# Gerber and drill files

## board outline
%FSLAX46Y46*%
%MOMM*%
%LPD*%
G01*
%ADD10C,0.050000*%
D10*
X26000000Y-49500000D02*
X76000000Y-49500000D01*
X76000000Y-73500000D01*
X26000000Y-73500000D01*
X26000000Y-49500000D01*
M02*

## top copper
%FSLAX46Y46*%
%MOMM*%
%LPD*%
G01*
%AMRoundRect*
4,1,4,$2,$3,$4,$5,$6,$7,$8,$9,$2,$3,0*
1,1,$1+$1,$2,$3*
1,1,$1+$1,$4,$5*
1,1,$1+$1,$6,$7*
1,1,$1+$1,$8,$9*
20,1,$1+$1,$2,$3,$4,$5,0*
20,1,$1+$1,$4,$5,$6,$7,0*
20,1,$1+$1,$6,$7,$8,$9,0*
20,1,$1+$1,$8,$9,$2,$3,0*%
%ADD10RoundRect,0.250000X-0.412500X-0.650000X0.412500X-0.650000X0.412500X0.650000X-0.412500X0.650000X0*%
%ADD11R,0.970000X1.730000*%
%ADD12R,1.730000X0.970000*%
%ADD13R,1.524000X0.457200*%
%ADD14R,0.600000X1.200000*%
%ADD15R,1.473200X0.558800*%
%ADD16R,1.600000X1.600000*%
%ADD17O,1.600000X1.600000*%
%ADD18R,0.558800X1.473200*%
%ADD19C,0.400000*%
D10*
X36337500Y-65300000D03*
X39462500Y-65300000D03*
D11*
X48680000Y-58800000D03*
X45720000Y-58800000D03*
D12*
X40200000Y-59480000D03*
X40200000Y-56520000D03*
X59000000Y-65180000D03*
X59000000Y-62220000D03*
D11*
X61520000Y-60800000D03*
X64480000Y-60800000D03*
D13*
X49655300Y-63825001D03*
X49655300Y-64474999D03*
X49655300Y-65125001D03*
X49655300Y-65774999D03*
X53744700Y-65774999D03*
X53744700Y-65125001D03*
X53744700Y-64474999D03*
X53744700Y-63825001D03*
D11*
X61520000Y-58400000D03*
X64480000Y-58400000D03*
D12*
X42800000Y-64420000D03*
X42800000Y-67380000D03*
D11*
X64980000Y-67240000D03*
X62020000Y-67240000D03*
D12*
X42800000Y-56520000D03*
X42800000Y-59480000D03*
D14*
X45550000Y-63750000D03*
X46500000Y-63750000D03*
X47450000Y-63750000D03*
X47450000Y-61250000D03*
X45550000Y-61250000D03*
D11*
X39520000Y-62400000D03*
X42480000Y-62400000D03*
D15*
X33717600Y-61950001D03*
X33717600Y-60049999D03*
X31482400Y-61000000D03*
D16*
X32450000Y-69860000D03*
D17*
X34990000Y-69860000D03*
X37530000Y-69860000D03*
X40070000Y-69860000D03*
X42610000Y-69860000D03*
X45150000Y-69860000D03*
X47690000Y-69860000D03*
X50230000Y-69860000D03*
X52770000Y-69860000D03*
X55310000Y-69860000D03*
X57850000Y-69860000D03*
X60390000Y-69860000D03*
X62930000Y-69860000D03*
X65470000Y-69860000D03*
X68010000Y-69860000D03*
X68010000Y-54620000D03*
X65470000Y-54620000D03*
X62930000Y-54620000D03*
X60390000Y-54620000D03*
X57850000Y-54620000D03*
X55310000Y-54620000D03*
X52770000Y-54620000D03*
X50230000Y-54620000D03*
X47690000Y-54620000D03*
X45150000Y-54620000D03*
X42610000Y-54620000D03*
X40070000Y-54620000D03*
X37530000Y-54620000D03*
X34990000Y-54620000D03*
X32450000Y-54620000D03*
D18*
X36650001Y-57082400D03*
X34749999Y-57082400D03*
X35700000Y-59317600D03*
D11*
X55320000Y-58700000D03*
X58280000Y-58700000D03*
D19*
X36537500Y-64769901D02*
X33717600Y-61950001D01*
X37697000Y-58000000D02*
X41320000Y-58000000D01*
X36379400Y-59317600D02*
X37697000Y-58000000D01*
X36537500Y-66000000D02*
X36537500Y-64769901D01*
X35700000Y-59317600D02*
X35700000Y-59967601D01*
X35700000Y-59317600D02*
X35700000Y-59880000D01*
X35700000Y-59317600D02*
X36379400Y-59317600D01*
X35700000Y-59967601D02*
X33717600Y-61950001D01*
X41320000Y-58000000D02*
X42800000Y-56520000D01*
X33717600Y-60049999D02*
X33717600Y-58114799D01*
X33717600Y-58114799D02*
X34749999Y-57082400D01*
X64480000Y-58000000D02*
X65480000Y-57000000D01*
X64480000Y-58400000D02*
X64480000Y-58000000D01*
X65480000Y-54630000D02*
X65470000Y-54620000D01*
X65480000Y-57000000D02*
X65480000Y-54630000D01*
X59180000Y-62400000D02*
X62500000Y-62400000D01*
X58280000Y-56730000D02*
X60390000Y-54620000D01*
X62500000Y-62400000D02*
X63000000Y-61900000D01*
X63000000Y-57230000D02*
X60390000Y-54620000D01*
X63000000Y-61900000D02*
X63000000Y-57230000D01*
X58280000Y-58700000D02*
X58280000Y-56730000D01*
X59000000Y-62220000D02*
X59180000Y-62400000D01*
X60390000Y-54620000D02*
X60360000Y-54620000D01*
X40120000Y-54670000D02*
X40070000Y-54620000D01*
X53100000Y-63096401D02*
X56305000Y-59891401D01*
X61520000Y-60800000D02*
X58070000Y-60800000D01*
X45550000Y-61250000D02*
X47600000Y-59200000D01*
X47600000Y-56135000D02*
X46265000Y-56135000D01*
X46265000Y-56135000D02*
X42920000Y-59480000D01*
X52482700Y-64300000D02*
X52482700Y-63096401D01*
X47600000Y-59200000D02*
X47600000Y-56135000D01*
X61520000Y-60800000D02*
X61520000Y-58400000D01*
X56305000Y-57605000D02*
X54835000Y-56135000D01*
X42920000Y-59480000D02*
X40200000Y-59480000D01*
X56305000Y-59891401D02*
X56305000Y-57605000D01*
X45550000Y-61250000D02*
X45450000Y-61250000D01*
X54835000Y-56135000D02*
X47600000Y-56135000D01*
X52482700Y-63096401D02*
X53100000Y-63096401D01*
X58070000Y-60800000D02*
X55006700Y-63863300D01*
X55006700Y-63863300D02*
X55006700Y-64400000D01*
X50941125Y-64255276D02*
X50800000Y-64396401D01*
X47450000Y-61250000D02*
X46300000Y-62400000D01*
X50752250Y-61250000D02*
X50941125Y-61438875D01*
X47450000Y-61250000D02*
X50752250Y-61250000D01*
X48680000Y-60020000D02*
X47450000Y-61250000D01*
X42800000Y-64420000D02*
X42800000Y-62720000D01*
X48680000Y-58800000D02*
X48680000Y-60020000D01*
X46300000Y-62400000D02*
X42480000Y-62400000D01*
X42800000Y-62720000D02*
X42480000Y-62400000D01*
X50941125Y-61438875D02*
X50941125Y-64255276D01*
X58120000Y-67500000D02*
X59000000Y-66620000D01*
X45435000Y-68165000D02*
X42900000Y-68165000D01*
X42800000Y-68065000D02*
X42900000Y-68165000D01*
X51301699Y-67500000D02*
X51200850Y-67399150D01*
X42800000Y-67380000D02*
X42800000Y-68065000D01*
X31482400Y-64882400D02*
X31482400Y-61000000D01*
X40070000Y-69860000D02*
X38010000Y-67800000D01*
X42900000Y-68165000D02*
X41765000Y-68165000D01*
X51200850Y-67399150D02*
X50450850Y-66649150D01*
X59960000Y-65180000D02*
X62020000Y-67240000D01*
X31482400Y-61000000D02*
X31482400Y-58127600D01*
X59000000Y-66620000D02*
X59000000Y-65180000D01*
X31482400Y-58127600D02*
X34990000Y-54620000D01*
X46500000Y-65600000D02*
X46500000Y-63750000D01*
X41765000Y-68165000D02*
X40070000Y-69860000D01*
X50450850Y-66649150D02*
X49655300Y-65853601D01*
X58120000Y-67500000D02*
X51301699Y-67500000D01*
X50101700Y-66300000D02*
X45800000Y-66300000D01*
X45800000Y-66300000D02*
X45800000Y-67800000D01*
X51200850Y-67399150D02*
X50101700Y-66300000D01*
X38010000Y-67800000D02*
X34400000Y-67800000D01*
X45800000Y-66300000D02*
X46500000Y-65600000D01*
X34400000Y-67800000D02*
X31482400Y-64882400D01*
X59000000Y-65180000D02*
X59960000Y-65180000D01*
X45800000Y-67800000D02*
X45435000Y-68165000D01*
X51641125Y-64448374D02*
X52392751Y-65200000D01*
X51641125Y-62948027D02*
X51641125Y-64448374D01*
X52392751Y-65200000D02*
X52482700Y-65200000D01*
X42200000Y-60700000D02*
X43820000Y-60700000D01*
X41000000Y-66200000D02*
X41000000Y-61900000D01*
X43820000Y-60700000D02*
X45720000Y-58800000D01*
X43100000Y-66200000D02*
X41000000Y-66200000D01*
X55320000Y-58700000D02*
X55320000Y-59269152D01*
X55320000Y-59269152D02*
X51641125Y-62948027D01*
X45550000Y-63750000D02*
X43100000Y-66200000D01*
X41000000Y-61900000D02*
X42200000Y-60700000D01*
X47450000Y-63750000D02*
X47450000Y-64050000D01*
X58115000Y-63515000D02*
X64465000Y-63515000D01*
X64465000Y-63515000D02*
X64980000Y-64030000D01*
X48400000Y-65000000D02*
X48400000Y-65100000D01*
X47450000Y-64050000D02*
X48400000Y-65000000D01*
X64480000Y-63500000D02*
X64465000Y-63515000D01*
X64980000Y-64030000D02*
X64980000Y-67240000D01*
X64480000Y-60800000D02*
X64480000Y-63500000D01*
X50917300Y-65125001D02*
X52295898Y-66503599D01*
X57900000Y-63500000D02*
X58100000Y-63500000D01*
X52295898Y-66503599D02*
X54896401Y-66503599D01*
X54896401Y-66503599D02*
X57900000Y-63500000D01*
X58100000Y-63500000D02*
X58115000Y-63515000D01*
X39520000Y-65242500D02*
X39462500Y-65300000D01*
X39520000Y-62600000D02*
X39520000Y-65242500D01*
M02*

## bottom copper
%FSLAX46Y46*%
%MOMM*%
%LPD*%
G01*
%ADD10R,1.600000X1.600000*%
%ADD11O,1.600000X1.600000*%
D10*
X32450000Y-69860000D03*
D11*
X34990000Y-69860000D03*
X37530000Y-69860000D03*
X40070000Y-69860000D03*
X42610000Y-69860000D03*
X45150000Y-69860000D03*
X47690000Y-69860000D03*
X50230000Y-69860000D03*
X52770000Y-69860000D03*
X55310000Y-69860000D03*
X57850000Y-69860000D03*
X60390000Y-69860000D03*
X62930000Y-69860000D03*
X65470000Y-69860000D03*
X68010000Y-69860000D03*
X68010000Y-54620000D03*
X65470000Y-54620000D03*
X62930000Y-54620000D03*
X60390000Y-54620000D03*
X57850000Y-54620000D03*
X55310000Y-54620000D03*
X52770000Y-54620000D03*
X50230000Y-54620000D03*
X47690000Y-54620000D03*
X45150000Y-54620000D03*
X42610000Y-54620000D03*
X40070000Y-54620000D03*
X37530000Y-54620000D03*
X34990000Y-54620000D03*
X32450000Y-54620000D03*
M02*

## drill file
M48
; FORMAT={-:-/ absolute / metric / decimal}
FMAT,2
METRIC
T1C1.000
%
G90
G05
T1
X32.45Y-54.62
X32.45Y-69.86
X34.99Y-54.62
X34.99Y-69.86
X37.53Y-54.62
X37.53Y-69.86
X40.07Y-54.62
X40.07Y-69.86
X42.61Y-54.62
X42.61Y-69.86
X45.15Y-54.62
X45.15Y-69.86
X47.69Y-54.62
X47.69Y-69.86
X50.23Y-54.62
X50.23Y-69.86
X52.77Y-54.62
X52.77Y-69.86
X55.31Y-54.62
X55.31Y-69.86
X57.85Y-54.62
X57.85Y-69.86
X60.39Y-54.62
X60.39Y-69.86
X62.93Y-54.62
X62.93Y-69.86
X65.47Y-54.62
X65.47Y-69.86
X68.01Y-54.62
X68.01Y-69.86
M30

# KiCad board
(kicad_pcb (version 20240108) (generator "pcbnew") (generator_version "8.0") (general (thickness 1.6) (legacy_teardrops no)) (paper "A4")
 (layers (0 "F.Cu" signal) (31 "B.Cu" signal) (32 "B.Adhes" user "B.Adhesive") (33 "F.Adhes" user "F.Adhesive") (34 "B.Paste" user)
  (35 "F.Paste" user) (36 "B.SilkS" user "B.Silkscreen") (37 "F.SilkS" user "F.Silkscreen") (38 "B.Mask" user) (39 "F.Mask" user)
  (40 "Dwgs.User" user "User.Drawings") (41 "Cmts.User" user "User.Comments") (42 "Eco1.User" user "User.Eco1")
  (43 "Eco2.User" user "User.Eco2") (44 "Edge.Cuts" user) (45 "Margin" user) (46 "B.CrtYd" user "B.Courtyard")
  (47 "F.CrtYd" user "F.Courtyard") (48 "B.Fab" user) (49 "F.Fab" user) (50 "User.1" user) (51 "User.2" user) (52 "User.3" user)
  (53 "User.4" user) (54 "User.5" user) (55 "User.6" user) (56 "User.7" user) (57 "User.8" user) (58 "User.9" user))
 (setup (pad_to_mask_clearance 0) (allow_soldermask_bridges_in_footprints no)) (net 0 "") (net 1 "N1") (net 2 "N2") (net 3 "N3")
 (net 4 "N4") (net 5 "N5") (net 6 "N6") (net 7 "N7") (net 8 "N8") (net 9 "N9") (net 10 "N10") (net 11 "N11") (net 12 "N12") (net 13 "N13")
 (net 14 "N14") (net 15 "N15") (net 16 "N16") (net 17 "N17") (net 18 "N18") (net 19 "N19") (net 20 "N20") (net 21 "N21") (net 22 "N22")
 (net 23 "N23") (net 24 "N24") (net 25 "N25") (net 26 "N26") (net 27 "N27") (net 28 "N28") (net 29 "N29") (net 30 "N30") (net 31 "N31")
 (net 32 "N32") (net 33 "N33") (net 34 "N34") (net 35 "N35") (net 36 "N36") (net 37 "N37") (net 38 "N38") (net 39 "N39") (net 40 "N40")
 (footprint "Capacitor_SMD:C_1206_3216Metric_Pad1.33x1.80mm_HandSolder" (layer "F.Cu") (at 37.9 65.3)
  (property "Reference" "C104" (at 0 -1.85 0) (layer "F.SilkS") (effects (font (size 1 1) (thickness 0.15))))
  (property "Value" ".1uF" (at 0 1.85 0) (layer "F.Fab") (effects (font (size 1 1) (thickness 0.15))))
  (pad "1" smd roundrect (at -1.5625 0) (size 1.325 1.8) (layers "F.Cu" "F.Paste" "F.Mask") (roundrect_rratio 0.188679) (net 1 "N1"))
  (pad "2" smd roundrect (at 1.5625 0) (size 1.325 1.8) (layers "F.Cu" "F.Paste" "F.Mask") (roundrect_rratio 0.188679) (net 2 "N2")))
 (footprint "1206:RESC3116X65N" (layer "F.Cu") (at 47.2 58.8 180)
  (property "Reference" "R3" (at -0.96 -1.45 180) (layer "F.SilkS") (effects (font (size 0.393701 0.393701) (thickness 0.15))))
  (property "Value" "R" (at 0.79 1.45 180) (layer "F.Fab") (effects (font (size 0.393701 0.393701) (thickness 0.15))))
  (pad "1" smd rect (at -1.48 0 180) (size 0.97 1.73) (layers "F.Cu" "F.Paste" "F.Mask") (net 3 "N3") (solder_mask_margin 0.102))
  (pad "2" smd rect (at 1.48 0 180) (size 0.97 1.73) (layers "F.Cu" "F.Paste" "F.Mask") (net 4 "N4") (solder_mask_margin 0.102)))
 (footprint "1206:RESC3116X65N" (layer "F.Cu") (at 40.2 58 90)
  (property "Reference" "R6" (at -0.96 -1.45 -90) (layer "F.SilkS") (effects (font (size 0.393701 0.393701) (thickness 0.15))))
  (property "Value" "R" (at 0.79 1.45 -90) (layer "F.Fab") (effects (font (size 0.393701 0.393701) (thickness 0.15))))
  (pad "1" smd rect (at -1.48 0 90) (size 0.97 1.73) (layers "F.Cu" "F.Paste" "F.Mask") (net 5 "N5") (solder_mask_margin 0.102))
  (pad "2" smd rect (at 1.48 0 90) (size 0.97 1.73) (layers "F.Cu" "F.Paste" "F.Mask") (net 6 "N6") (solder_mask_margin 0.102)))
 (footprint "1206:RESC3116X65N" (layer "F.Cu") (at 59 63.7 90)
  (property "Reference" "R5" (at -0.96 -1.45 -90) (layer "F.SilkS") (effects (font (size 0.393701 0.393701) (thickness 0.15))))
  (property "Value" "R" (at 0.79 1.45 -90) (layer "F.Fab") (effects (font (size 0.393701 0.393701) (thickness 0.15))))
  (pad "1" smd rect (at -1.48 0 90) (size 0.97 1.73) (layers "F.Cu" "F.Paste" "F.Mask") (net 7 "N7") (solder_mask_margin 0.102))
  (pad "2" smd rect (at 1.48 0 90) (size 0.97 1.73) (layers "F.Cu" "F.Paste" "F.Mask") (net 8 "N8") (solder_mask_margin 0.102)))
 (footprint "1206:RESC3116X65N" (layer "F.Cu") (at 63 60.8)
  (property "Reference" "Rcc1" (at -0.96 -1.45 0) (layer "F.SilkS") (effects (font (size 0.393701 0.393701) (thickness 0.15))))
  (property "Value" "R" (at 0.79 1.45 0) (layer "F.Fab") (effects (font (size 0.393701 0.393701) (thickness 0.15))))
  (pad "1" smd rect (at -1.48 0) (size 0.97 1.73) (layers "F.Cu" "F.Paste" "F.Mask") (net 5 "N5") (solder_mask_margin 0.102))
  (pad "2" smd rect (at 1.48 0) (size 0.97 1.73) (layers "F.Cu" "F.Paste" "F.Mask") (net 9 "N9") (solder_mask_margin 0.102)))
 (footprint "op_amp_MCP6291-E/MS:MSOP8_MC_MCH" (layer "F.Cu") (at 51.7 64.8)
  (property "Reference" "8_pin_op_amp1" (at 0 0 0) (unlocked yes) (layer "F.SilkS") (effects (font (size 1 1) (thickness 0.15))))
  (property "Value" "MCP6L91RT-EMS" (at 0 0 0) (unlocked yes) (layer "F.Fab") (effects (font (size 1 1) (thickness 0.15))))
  (pad "1" smd rect (at -2.0447 -0.974999) (size 1.524 0.4572) (layers "F.Cu" "F.Paste" "F.Mask") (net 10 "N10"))
  (pad "2" smd rect (at -2.0447 -0.325001) (size 1.524 0.4572) (layers "F.Cu" "F.Paste" "F.Mask") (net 3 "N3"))
  (pad "3" smd rect (at -2.0447 0.325001) (size 1.524 0.4572) (layers "F.Cu" "F.Paste" "F.Mask") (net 9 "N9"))
  (pad "4" smd rect (at -2.0447 0.974999) (size 1.524 0.4572) (layers "F.Cu" "F.Paste" "F.Mask") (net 7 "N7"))
  (pad "5" smd rect (at 2.0447 0.974999) (size 1.524 0.4572) (layers "F.Cu" "F.Paste" "F.Mask") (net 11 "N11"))
  (pad "6" smd rect (at 2.0447 0.325001) (size 1.524 0.4572) (layers "F.Cu" "F.Paste" "F.Mask") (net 4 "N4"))
  (pad "7" smd rect (at 2.0447 -0.325001) (size 1.524 0.4572) (layers "F.Cu" "F.Paste" "F.Mask") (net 5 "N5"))
  (pad "8" smd rect (at 2.0447 -0.974999) (size 1.524 0.4572) (layers "F.Cu" "F.Paste" "F.Mask") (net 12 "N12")))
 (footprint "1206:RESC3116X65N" (layer "F.Cu") (at 63 58.4)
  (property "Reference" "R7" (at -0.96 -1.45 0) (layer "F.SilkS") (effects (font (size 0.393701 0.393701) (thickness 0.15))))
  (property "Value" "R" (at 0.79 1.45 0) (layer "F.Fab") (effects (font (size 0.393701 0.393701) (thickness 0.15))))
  (pad "1" smd rect (at -1.48 0) (size 0.97 1.73) (layers "F.Cu" "F.Paste" "F.Mask") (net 5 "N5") (solder_mask_margin 0.102))
  (pad "2" smd rect (at 1.48 0) (size 0.97 1.73) (layers "F.Cu" "F.Paste" "F.Mask") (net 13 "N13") (solder_mask_margin 0.102)))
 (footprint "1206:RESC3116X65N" (layer "F.Cu") (at 42.8 65.9 -90)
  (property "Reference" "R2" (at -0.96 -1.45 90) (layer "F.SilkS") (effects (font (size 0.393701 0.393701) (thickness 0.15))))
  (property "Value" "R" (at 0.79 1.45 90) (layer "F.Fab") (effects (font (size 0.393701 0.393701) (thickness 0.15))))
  (pad "1" smd rect (at -1.48 0 270) (size 0.97 1.73) (layers "F.Cu" "F.Paste" "F.Mask") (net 3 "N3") (solder_mask_margin 0.102))
  (pad "2" smd rect (at 1.48 0 270) (size 0.97 1.73) (layers "F.Cu" "F.Paste" "F.Mask") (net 7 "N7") (solder_mask_margin 0.102)))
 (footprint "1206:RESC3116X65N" (layer "F.Cu") (at 63.5 67.24 180)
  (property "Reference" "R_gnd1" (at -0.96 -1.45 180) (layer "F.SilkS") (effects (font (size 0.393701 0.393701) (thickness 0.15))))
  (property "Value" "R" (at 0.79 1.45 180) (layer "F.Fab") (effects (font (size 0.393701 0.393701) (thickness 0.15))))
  (pad "1" smd rect (at -1.48 0 180) (size 0.97 1.73) (layers "F.Cu" "F.Paste" "F.Mask") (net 9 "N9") (solder_mask_margin 0.102))
  (pad "2" smd rect (at 1.48 0 180) (size 0.97 1.73) (layers "F.Cu" "F.Paste" "F.Mask") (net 7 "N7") (solder_mask_margin 0.102)))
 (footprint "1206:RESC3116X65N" (layer "F.Cu") (at 42.8 58 -90)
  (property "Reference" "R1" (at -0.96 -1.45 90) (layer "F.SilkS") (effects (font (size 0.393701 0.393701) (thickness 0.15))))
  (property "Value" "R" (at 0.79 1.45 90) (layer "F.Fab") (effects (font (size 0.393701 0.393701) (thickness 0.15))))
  (pad "1" smd rect (at -1.48 0 270) (size 0.97 1.73) (layers "F.Cu" "F.Paste" "F.Mask") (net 1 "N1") (solder_mask_margin 0.102))
  (pad "2" smd rect (at 1.48 0 270) (size 0.97 1.73) (layers "F.Cu" "F.Paste" "F.Mask") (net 5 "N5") (solder_mask_margin 0.102)))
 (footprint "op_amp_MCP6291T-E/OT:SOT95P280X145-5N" (layer "F.Cu") (at 46.5 62.5 90)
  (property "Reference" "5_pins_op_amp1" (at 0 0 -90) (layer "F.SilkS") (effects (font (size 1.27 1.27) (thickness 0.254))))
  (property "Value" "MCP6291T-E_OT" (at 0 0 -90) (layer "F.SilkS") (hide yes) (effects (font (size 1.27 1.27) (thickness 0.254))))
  (pad "1" smd rect (at -1.25 -0.95 180) (size 0.6 1.2) (layers "F.Cu" "F.Paste" "F.Mask") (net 4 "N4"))
  (pad "2" smd rect (at -1.25 0 180) (size 0.6 1.2) (layers "F.Cu" "F.Paste" "F.Mask") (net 7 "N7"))
  (pad "3" smd rect (at -1.25 0.95 180) (size 0.6 1.2) (layers "F.Cu" "F.Paste" "F.Mask") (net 9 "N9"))
  (pad "4" smd rect (at 1.25 0.95 180) (size 0.6 1.2) (layers "F.Cu" "F.Paste" "F.Mask") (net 3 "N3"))
  (pad "5" smd rect (at 1.25 -0.95 180) (size 0.6 1.2) (layers "F.Cu" "F.Paste" "F.Mask") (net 5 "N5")))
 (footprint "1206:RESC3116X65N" (layer "F.Cu") (at 41 62.4)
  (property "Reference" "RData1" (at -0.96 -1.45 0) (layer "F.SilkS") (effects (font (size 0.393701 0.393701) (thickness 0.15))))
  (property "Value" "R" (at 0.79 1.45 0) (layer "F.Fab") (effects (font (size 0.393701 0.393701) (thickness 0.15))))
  (pad "1" smd rect (at -1.48 0) (size 0.97 1.73) (layers "F.Cu" "F.Paste" "F.Mask") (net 2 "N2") (solder_mask_margin 0.102))
  (pad "2" smd rect (at 1.48 0) (size 0.97 1.73) (layers "F.Cu" "F.Paste" "F.Mask") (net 3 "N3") (solder_mask_margin 0.102)))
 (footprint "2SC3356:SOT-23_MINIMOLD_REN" (layer "F.Cu") (at 32.6 61 90)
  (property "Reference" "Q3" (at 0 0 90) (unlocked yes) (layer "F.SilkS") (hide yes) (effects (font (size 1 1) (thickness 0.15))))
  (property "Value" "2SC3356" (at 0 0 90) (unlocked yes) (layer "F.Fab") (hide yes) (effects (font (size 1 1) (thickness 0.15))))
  (pad "1" smd rect (at -0.950001 1.1176 90) (size 0.5588 1.4732) (layers "F.Cu" "F.Paste" "F.Mask") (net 1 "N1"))
  (pad "2" smd rect (at 0.950001 1.1176 90) (size 0.5588 1.4732) (layers "F.Cu" "F.Paste" "F.Mask") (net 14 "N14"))
  (pad "3" smd rect (at 0 -1.1176 90) (size 0.5588 1.4732) (layers "F.Cu" "F.Paste" "F.Mask") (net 7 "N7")))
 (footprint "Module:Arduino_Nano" (layer "F.Cu") (at 32.45 69.86 90)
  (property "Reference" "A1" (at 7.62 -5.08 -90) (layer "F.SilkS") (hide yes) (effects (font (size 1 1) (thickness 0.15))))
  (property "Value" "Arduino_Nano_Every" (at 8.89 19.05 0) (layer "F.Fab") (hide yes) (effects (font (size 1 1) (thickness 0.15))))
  (pad "1" thru_hole rect (at 0 0 90) (size 1.6 1.6) (drill 1) (layers "*.Cu" "*.Mask") (remove_unused_layers no) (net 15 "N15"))
  (pad "2" thru_hole oval (at 0 2.54 90) (size 1.6 1.6) (drill 1) (layers "*.Cu" "*.Mask") (remove_unused_layers no) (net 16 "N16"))
  (pad "3" thru_hole oval (at 0 5.08 90) (size 1.6 1.6) (drill 1) (layers "*.Cu" "*.Mask") (remove_unused_layers no) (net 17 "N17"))
  (pad "4" thru_hole oval (at 0 7.62 90) (size 1.6 1.6) (drill 1) (layers "*.Cu" "*.Mask") (remove_unused_layers no) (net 7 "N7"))
  (pad "5" thru_hole oval (at 0 10.16 90) (size 1.6 1.6) (drill 1) (layers "*.Cu" "*.Mask") (remove_unused_layers no) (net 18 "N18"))
  (pad "6" thru_hole oval (at 0 12.7 90) (size 1.6 1.6) (drill 1) (layers "*.Cu" "*.Mask") (remove_unused_layers no) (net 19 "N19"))
  (pad "7" thru_hole oval (at 0 15.24 90) (size 1.6 1.6) (drill 1) (layers "*.Cu" "*.Mask") (remove_unused_layers no) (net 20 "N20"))
  (pad "8" thru_hole oval (at 0 17.78 90) (size 1.6 1.6) (drill 1) (layers "*.Cu" "*.Mask") (remove_unused_layers no) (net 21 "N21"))
  (pad "9" thru_hole oval (at 0 20.32 90) (size 1.6 1.6) (drill 1) (layers "*.Cu" "*.Mask") (remove_unused_layers no) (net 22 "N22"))
  (pad "10" thru_hole oval (at 0 22.86 90) (size 1.6 1.6) (drill 1) (layers "*.Cu" "*.Mask") (remove_unused_layers no) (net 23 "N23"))
  (pad "11" thru_hole oval (at 0 25.4 90) (size 1.6 1.6) (drill 1) (layers "*.Cu" "*.Mask") (remove_unused_layers no) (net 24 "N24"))
  (pad "12" thru_hole oval (at 0 27.94 90) (size 1.6 1.6) (drill 1) (layers "*.Cu" "*.Mask") (remove_unused_layers no) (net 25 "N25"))
  (pad "13" thru_hole oval (at 0 30.48 90) (size 1.6 1.6) (drill 1) (layers "*.Cu" "*.Mask") (remove_unused_layers no) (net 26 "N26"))
  (pad "14" thru_hole oval (at 0 33.02 90) (size 1.6 1.6) (drill 1) (layers "*.Cu" "*.Mask") (remove_unused_layers no) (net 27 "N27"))
  (pad "15" thru_hole oval (at 0 35.56 90) (size 1.6 1.6) (drill 1) (layers "*.Cu" "*.Mask") (remove_unused_layers no) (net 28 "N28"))
  (pad "16" thru_hole oval (at 15.24 35.56 90) (size 1.6 1.6) (drill 1) (layers "*.Cu" "*.Mask") (remove_unused_layers no) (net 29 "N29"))
  (pad "17" thru_hole oval (at 15.24 33.02 90) (size 1.6 1.6) (drill 1) (layers "*.Cu" "*.Mask") (remove_unused_layers no) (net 13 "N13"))
  (pad "18" thru_hole oval (at 15.24 30.48 90) (size 1.6 1.6) (drill 1) (layers "*.Cu" "*.Mask") (remove_unused_layers no) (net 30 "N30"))
  (pad "19" thru_hole oval (at 15.24 27.94 90) (size 1.6 1.6) (drill 1) (layers "*.Cu" "*.Mask") (remove_unused_layers no) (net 8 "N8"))
  (pad "20" thru_hole oval (at 15.24 25.4 90) (size 1.6 1.6) (drill 1) (layers "*.Cu" "*.Mask") (remove_unused_layers no) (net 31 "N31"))
  (pad "21" thru_hole oval (at 15.24 22.86 90) (size 1.6 1.6) (drill 1) (layers "*.Cu" "*.Mask") (remove_unused_layers no) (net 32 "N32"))
  (pad "22" thru_hole oval (at 15.24 20.32 90) (size 1.6 1.6) (drill 1) (layers "*.Cu" "*.Mask") (remove_unused_layers no) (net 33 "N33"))
  (pad "23" thru_hole oval (at 15.24 17.78 90) (size 1.6 1.6) (drill 1) (layers "*.Cu" "*.Mask") (remove_unused_layers no) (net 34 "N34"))
  (pad "24" thru_hole oval (at 15.24 15.24 90) (size 1.6 1.6) (drill 1) (layers "*.Cu" "*.Mask") (remove_unused_layers no) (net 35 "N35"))
  (pad "25" thru_hole oval (at 15.24 12.7 90) (size 1.6 1.6) (drill 1) (layers "*.Cu" "*.Mask") (remove_unused_layers no) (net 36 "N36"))
  (pad "26" thru_hole oval (at 15.24 10.16 90) (size 1.6 1.6) (drill 1) (layers "*.Cu" "*.Mask") (remove_unused_layers no) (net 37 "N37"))
  (pad "27" thru_hole oval (at 15.24 7.62 90) (size 1.6 1.6) (drill 1) (layers "*.Cu" "*.Mask") (remove_unused_layers no) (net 6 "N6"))
  (pad "28" thru_hole oval (at 15.24 5.08 90) (size 1.6 1.6) (drill 1) (layers "*.Cu" "*.Mask") (remove_unused_layers no) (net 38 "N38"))
  (pad "29" thru_hole oval (at 15.24 2.54 90) (size 1.6 1.6) (drill 1) (layers "*.Cu" "*.Mask") (remove_unused_layers no) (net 7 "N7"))
  (pad "30" thru_hole oval (at 15.24 0 90) (size 1.6 1.6) (drill 1) (layers "*.Cu" "*.Mask") (remove_unused_layers no) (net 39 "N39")))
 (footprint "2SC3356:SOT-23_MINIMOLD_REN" (layer "F.Cu") (at 35.7 58.2 180)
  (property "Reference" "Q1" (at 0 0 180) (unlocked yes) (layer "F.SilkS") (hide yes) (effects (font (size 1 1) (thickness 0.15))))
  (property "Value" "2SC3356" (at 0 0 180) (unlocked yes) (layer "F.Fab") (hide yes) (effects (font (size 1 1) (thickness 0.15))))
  (pad "1" smd rect (at -0.950001 1.1176 180) (size 0.5588 1.4732) (layers "F.Cu" "F.Paste" "F.Mask") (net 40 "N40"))
  (pad "2" smd rect (at 0.950001 1.1176 180) (size 0.5588 1.4732) (layers "F.Cu" "F.Paste" "F.Mask") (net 14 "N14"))
  (pad "3" smd rect (at 0 -1.1176 180) (size 0.5588 1.4732) (layers "F.Cu" "F.Paste" "F.Mask") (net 1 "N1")))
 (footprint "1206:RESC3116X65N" (layer "F.Cu") (at 56.8 58.7)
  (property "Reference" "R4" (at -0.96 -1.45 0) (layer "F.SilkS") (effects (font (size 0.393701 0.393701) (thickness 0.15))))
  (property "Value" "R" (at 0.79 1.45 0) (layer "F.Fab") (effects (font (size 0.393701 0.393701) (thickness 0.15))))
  (pad "1" smd rect (at -1.48 0) (size 0.97 1.73) (layers "F.Cu" "F.Paste" "F.Mask") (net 4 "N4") (solder_mask_margin 0.102))
  (pad "2" smd rect (at 1.48 0) (size 0.97 1.73) (layers "F.Cu" "F.Paste" "F.Mask") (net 8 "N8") (solder_mask_margin 0.102)))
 (gr_rect (start 26 49.5) (end 76 73.5) (stroke (width 0.05) (type default)) (fill none) (layer "Edge.Cuts"))
 (segment (start 36.5375 64.769901) (end 33.7176 61.950001) (width 0.4) (layer "F.Cu") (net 1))
 (segment (start 37.697 58) (end 41.32 58) (width 0.4) (layer "F.Cu") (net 1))
 (segment (start 36.3794 59.3176) (end 37.697 58) (width 0.4) (layer "F.Cu") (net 1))
 (segment (start 36.5375 66) (end 36.5375 64.769901) (width 0.4) (layer "F.Cu") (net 1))
 (segment (start 35.7 59.3176) (end 35.7 59.967601) (width 0.4) (layer "F.Cu") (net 1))
 (segment (start 35.7 59.3176) (end 35.7 59.88) (width 0.4) (layer "F.Cu") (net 1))
 (segment (start 35.7 59.3176) (end 36.3794 59.3176) (width 0.4) (layer "F.Cu") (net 1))
 (segment (start 35.7 59.967601) (end 33.7176 61.950001) (width 0.4) (layer "F.Cu") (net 1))
 (segment (start 41.32 58) (end 42.8 56.52) (width 0.4) (layer "F.Cu") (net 1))
 (segment (start 33.7176 60.049999) (end 33.7176 58.114799) (width 0.4) (layer "F.Cu") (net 14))
 (segment (start 33.7176 58.114799) (end 34.749999 57.0824) (width 0.4) (layer "F.Cu") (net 14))
 (segment (start 64.48 58) (end 65.48 57) (width 0.4) (layer "F.Cu") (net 13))
 (segment (start 64.48 58.4) (end 64.48 58) (width 0.4) (layer "F.Cu") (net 13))
 (segment (start 65.48 54.63) (end 65.47 54.62) (width 0.4) (layer "F.Cu") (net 13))
 (segment (start 65.48 57) (end 65.48 54.63) (width 0.4) (layer "F.Cu") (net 13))
 (segment (start 59.18 62.4) (end 62.5 62.4) (width 0.4) (layer "F.Cu") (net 8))
 (segment (start 58.28 56.73) (end 60.39 54.62) (width 0.4) (layer "F.Cu") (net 8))
 (segment (start 62.5 62.4) (end 63 61.9) (width 0.4) (layer "F.Cu") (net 8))
 (segment (start 63 57.23) (end 60.39 54.62) (width 0.4) (layer "F.Cu") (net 8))
 (segment (start 63 61.9) (end 63 57.23) (width 0.4) (layer "F.Cu") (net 8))
 (segment (start 58.28 58.7) (end 58.28 56.73) (width 0.4) (layer "F.Cu") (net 8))
 (segment (start 59 62.22) (end 59.18 62.4) (width 0.4) (layer "F.Cu") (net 8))
 (segment (start 60.39 54.62) (end 60.36 54.62) (width 0.4) (layer "F.Cu") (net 8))
 (segment (start 40.12 54.67) (end 40.07 54.62) (width 0.4) (layer "F.Cu") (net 6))
 (segment (start 53.1 63.096401) (end 56.305 59.891401) (width 0.4) (layer "F.Cu") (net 5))
 (segment (start 61.52 60.8) (end 58.07 60.8) (width 0.4) (layer "F.Cu") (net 5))
 (segment (start 45.55 61.25) (end 47.6 59.2) (width 0.4) (layer "F.Cu") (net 5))
 (segment (start 47.6 56.135) (end 46.265 56.135) (width 0.4) (layer "F.Cu") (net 5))
 (segment (start 46.265 56.135) (end 42.92 59.48) (width 0.4) (layer "F.Cu") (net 5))
 (segment (start 52.4827 64.3) (end 52.4827 63.096401) (width 0.4) (layer "F.Cu") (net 5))
 (segment (start 47.6 59.2) (end 47.6 56.135) (width 0.4) (layer "F.Cu") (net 5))
 (segment (start 61.52 60.8) (end 61.52 58.4) (width 0.4) (layer "F.Cu") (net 5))
 (segment (start 56.305 57.605) (end 54.835 56.135) (width 0.4) (layer "F.Cu") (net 5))
 (segment (start 42.92 59.48) (end 40.2 59.48) (width 0.4) (layer "F.Cu") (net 5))
 (segment (start 56.305 59.891401) (end 56.305 57.605) (width 0.4) (layer "F.Cu") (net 5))
 (segment (start 45.55 61.25) (end 45.45 61.25) (width 0.4) (layer "F.Cu") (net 5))
 (segment (start 54.835 56.135) (end 47.6 56.135) (width 0.4) (layer "F.Cu") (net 5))
 (segment (start 52.4827 63.096401) (end 53.1 63.096401) (width 0.4) (layer "F.Cu") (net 5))
 (segment (start 58.07 60.8) (end 55.0067 63.8633) (width 0.4) (layer "F.Cu") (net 5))
 (segment (start 55.0067 63.8633) (end 55.0067 64.4) (width 0.4) (layer "F.Cu") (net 5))
 (segment (start 50.941125 64.255276) (end 50.8 64.396401) (width 0.4) (layer "F.Cu") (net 3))
 (segment (start 47.45 61.25) (end 46.3 62.4) (width 0.4) (layer "F.Cu") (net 3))
 (segment (start 50.75225 61.25) (end 50.941125 61.438875) (width 0.4) (layer "F.Cu") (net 3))
 (segment (start 47.45 61.25) (end 50.75225 61.25) (width 0.4) (layer "F.Cu") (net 3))
 (segment (start 48.68 60.02) (end 47.45 61.25) (width 0.4) (layer "F.Cu") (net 3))
 (segment (start 42.8 64.42) (end 42.8 62.72) (width 0.4) (layer "F.Cu") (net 3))
 (segment (start 48.68 58.8) (end 48.68 60.02) (width 0.4) (layer "F.Cu") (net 3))
 (segment (start 46.3 62.4) (end 42.48 62.4) (width 0.4) (layer "F.Cu") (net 3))
 (segment (start 42.8 62.72) (end 42.48 62.4) (width 0.4) (layer "F.Cu") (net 3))
 (segment (start 50.941125 61.438875) (end 50.941125 64.255276) (width 0.4) (layer "F.Cu") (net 3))
 (segment (start 58.12 67.5) (end 59 66.62) (width 0.4) (layer "F.Cu") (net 7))
 (segment (start 45.435 68.165) (end 42.9 68.165) (width 0.4) (layer "F.Cu") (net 7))
 (segment (start 42.8 68.065) (end 42.9 68.165) (width 0.4) (layer "F.Cu") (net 7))
 (segment (start 51.301699 67.5) (end 51.20085 67.39915) (width 0.4) (layer "F.Cu") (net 7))
 (segment (start 42.8 67.38) (end 42.8 68.065) (width 0.4) (layer "F.Cu") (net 7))
 (segment (start 31.4824 64.8824) (end 31.4824 61) (width 0.4) (layer "F.Cu") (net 7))
 (segment (start 40.07 69.86) (end 38.01 67.8) (width 0.4) (layer "F.Cu") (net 7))
 (segment (start 42.9 68.165) (end 41.765 68.165) (width 0.4) (layer "F.Cu") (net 7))
 (segment (start 51.20085 67.39915) (end 50.45085 66.64915) (width 0.4) (layer "F.Cu") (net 7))
 (segment (start 59.96 65.18) (end 62.02 67.24) (width 0.4) (layer "F.Cu") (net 7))
 (segment (start 31.4824 61) (end 31.4824 58.1276) (width 0.4) (layer "F.Cu") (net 7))
 (segment (start 59 66.62) (end 59 65.18) (width 0.4) (layer "F.Cu") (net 7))
 (segment (start 31.4824 58.1276) (end 34.99 54.62) (width 0.4) (layer "F.Cu") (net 7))
 (segment (start 46.5 65.6) (end 46.5 63.75) (width 0.4) (layer "F.Cu") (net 7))
 (segment (start 41.765 68.165) (end 40.07 69.86) (width 0.4) (layer "F.Cu") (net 7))
 (segment (start 50.45085 66.64915) (end 49.6553 65.853601) (width 0.4) (layer "F.Cu") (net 7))
 (segment (start 58.12 67.5) (end 51.301699 67.5) (width 0.4) (layer "F.Cu") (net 7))
 (segment (start 50.1017 66.3) (end 45.8 66.3) (width 0.4) (layer "F.Cu") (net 7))
 (segment (start 45.8 66.3) (end 45.8 67.8) (width 0.4) (layer "F.Cu") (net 7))
 (segment (start 51.20085 67.39915) (end 50.1017 66.3) (width 0.4) (layer "F.Cu") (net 7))
 (segment (start 38.01 67.8) (end 34.4 67.8) (width 0.4) (layer "F.Cu") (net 7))
 (segment (start 45.8 66.3) (end 46.5 65.6) (width 0.4) (layer "F.Cu") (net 7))
 (segment (start 34.4 67.8) (end 31.4824 64.8824) (width 0.4) (layer "F.Cu") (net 7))
 (segment (start 59 65.18) (end 59.96 65.18) (width 0.4) (layer "F.Cu") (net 7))
 (segment (start 45.8 67.8) (end 45.435 68.165) (width 0.4) (layer "F.Cu") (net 7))
 (segment (start 51.641125 64.448374) (end 52.392751 65.2) (width 0.4) (layer "F.Cu") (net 4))
 (segment (start 51.641125 62.948027) (end 51.641125 64.448374) (width 0.4) (layer "F.Cu") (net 4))
 (segment (start 52.392751 65.2) (end 52.4827 65.2) (width 0.4) (layer "F.Cu") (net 4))
 (segment (start 42.2 60.7) (end 43.82 60.7) (width 0.4) (layer "F.Cu") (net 4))
 (segment (start 41 66.2) (end 41 61.9) (width 0.4) (layer "F.Cu") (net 4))
 (segment (start 43.82 60.7) (end 45.72 58.8) (width 0.4) (layer "F.Cu") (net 4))
 (segment (start 43.1 66.2) (end 41 66.2) (width 0.4) (layer "F.Cu") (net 4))
 (segment (start 55.32 58.7) (end 55.32 59.269152) (width 0.4) (layer "F.Cu") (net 4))
 (segment (start 55.32 59.269152) (end 51.641125 62.948027) (width 0.4) (layer "F.Cu") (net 4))
 (segment (start 45.55 63.75) (end 43.1 66.2) (width 0.4) (layer "F.Cu") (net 4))
 (segment (start 41 61.9) (end 42.2 60.7) (width 0.4) (layer "F.Cu") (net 4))
 (segment (start 47.45 63.75) (end 47.45 64.05) (width 0.4) (layer "F.Cu") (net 9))
 (segment (start 58.115 63.515) (end 64.465 63.515) (width 0.4) (layer "F.Cu") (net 9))
 (segment (start 64.465 63.515) (end 64.98 64.03) (width 0.4) (layer "F.Cu") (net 9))
 (segment (start 48.4 65) (end 48.4 65.1) (width 0.4) (layer "F.Cu") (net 9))
 (segment (start 47.45 64.05) (end 48.4 65) (width 0.4) (layer "F.Cu") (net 9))
 (segment (start 64.48 63.5) (end 64.465 63.515) (width 0.4) (layer "F.Cu") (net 9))
 (segment (start 64.98 64.03) (end 64.98 67.24) (width 0.4) (layer "F.Cu") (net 9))
 (segment (start 64.48 60.8) (end 64.48 63.5) (width 0.4) (layer "F.Cu") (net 9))
 (segment (start 50.9173 65.125001) (end 52.295898 66.503599) (width 0.4) (layer "F.Cu") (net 9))
 (segment (start 57.9 63.5) (end 58.1 63.5) (width 0.4) (layer "F.Cu") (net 9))
 (segment (start 52.295898 66.503599) (end 54.896401 66.503599) (width 0.4) (layer "F.Cu") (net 9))
 (segment (start 54.896401 66.503599) (end 57.9 63.5) (width 0.4) (layer "F.Cu") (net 9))
 (segment (start 58.1 63.5) (end 58.115 63.515) (width 0.4) (layer "F.Cu") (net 9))
 (segment (start 39.52 65.2425) (end 39.4625 65.3) (width 0.4) (layer "F.Cu") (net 2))
 (segment (start 39.52 62.6) (end 39.52 65.2425) (width 0.4) (layer "F.Cu") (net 2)))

